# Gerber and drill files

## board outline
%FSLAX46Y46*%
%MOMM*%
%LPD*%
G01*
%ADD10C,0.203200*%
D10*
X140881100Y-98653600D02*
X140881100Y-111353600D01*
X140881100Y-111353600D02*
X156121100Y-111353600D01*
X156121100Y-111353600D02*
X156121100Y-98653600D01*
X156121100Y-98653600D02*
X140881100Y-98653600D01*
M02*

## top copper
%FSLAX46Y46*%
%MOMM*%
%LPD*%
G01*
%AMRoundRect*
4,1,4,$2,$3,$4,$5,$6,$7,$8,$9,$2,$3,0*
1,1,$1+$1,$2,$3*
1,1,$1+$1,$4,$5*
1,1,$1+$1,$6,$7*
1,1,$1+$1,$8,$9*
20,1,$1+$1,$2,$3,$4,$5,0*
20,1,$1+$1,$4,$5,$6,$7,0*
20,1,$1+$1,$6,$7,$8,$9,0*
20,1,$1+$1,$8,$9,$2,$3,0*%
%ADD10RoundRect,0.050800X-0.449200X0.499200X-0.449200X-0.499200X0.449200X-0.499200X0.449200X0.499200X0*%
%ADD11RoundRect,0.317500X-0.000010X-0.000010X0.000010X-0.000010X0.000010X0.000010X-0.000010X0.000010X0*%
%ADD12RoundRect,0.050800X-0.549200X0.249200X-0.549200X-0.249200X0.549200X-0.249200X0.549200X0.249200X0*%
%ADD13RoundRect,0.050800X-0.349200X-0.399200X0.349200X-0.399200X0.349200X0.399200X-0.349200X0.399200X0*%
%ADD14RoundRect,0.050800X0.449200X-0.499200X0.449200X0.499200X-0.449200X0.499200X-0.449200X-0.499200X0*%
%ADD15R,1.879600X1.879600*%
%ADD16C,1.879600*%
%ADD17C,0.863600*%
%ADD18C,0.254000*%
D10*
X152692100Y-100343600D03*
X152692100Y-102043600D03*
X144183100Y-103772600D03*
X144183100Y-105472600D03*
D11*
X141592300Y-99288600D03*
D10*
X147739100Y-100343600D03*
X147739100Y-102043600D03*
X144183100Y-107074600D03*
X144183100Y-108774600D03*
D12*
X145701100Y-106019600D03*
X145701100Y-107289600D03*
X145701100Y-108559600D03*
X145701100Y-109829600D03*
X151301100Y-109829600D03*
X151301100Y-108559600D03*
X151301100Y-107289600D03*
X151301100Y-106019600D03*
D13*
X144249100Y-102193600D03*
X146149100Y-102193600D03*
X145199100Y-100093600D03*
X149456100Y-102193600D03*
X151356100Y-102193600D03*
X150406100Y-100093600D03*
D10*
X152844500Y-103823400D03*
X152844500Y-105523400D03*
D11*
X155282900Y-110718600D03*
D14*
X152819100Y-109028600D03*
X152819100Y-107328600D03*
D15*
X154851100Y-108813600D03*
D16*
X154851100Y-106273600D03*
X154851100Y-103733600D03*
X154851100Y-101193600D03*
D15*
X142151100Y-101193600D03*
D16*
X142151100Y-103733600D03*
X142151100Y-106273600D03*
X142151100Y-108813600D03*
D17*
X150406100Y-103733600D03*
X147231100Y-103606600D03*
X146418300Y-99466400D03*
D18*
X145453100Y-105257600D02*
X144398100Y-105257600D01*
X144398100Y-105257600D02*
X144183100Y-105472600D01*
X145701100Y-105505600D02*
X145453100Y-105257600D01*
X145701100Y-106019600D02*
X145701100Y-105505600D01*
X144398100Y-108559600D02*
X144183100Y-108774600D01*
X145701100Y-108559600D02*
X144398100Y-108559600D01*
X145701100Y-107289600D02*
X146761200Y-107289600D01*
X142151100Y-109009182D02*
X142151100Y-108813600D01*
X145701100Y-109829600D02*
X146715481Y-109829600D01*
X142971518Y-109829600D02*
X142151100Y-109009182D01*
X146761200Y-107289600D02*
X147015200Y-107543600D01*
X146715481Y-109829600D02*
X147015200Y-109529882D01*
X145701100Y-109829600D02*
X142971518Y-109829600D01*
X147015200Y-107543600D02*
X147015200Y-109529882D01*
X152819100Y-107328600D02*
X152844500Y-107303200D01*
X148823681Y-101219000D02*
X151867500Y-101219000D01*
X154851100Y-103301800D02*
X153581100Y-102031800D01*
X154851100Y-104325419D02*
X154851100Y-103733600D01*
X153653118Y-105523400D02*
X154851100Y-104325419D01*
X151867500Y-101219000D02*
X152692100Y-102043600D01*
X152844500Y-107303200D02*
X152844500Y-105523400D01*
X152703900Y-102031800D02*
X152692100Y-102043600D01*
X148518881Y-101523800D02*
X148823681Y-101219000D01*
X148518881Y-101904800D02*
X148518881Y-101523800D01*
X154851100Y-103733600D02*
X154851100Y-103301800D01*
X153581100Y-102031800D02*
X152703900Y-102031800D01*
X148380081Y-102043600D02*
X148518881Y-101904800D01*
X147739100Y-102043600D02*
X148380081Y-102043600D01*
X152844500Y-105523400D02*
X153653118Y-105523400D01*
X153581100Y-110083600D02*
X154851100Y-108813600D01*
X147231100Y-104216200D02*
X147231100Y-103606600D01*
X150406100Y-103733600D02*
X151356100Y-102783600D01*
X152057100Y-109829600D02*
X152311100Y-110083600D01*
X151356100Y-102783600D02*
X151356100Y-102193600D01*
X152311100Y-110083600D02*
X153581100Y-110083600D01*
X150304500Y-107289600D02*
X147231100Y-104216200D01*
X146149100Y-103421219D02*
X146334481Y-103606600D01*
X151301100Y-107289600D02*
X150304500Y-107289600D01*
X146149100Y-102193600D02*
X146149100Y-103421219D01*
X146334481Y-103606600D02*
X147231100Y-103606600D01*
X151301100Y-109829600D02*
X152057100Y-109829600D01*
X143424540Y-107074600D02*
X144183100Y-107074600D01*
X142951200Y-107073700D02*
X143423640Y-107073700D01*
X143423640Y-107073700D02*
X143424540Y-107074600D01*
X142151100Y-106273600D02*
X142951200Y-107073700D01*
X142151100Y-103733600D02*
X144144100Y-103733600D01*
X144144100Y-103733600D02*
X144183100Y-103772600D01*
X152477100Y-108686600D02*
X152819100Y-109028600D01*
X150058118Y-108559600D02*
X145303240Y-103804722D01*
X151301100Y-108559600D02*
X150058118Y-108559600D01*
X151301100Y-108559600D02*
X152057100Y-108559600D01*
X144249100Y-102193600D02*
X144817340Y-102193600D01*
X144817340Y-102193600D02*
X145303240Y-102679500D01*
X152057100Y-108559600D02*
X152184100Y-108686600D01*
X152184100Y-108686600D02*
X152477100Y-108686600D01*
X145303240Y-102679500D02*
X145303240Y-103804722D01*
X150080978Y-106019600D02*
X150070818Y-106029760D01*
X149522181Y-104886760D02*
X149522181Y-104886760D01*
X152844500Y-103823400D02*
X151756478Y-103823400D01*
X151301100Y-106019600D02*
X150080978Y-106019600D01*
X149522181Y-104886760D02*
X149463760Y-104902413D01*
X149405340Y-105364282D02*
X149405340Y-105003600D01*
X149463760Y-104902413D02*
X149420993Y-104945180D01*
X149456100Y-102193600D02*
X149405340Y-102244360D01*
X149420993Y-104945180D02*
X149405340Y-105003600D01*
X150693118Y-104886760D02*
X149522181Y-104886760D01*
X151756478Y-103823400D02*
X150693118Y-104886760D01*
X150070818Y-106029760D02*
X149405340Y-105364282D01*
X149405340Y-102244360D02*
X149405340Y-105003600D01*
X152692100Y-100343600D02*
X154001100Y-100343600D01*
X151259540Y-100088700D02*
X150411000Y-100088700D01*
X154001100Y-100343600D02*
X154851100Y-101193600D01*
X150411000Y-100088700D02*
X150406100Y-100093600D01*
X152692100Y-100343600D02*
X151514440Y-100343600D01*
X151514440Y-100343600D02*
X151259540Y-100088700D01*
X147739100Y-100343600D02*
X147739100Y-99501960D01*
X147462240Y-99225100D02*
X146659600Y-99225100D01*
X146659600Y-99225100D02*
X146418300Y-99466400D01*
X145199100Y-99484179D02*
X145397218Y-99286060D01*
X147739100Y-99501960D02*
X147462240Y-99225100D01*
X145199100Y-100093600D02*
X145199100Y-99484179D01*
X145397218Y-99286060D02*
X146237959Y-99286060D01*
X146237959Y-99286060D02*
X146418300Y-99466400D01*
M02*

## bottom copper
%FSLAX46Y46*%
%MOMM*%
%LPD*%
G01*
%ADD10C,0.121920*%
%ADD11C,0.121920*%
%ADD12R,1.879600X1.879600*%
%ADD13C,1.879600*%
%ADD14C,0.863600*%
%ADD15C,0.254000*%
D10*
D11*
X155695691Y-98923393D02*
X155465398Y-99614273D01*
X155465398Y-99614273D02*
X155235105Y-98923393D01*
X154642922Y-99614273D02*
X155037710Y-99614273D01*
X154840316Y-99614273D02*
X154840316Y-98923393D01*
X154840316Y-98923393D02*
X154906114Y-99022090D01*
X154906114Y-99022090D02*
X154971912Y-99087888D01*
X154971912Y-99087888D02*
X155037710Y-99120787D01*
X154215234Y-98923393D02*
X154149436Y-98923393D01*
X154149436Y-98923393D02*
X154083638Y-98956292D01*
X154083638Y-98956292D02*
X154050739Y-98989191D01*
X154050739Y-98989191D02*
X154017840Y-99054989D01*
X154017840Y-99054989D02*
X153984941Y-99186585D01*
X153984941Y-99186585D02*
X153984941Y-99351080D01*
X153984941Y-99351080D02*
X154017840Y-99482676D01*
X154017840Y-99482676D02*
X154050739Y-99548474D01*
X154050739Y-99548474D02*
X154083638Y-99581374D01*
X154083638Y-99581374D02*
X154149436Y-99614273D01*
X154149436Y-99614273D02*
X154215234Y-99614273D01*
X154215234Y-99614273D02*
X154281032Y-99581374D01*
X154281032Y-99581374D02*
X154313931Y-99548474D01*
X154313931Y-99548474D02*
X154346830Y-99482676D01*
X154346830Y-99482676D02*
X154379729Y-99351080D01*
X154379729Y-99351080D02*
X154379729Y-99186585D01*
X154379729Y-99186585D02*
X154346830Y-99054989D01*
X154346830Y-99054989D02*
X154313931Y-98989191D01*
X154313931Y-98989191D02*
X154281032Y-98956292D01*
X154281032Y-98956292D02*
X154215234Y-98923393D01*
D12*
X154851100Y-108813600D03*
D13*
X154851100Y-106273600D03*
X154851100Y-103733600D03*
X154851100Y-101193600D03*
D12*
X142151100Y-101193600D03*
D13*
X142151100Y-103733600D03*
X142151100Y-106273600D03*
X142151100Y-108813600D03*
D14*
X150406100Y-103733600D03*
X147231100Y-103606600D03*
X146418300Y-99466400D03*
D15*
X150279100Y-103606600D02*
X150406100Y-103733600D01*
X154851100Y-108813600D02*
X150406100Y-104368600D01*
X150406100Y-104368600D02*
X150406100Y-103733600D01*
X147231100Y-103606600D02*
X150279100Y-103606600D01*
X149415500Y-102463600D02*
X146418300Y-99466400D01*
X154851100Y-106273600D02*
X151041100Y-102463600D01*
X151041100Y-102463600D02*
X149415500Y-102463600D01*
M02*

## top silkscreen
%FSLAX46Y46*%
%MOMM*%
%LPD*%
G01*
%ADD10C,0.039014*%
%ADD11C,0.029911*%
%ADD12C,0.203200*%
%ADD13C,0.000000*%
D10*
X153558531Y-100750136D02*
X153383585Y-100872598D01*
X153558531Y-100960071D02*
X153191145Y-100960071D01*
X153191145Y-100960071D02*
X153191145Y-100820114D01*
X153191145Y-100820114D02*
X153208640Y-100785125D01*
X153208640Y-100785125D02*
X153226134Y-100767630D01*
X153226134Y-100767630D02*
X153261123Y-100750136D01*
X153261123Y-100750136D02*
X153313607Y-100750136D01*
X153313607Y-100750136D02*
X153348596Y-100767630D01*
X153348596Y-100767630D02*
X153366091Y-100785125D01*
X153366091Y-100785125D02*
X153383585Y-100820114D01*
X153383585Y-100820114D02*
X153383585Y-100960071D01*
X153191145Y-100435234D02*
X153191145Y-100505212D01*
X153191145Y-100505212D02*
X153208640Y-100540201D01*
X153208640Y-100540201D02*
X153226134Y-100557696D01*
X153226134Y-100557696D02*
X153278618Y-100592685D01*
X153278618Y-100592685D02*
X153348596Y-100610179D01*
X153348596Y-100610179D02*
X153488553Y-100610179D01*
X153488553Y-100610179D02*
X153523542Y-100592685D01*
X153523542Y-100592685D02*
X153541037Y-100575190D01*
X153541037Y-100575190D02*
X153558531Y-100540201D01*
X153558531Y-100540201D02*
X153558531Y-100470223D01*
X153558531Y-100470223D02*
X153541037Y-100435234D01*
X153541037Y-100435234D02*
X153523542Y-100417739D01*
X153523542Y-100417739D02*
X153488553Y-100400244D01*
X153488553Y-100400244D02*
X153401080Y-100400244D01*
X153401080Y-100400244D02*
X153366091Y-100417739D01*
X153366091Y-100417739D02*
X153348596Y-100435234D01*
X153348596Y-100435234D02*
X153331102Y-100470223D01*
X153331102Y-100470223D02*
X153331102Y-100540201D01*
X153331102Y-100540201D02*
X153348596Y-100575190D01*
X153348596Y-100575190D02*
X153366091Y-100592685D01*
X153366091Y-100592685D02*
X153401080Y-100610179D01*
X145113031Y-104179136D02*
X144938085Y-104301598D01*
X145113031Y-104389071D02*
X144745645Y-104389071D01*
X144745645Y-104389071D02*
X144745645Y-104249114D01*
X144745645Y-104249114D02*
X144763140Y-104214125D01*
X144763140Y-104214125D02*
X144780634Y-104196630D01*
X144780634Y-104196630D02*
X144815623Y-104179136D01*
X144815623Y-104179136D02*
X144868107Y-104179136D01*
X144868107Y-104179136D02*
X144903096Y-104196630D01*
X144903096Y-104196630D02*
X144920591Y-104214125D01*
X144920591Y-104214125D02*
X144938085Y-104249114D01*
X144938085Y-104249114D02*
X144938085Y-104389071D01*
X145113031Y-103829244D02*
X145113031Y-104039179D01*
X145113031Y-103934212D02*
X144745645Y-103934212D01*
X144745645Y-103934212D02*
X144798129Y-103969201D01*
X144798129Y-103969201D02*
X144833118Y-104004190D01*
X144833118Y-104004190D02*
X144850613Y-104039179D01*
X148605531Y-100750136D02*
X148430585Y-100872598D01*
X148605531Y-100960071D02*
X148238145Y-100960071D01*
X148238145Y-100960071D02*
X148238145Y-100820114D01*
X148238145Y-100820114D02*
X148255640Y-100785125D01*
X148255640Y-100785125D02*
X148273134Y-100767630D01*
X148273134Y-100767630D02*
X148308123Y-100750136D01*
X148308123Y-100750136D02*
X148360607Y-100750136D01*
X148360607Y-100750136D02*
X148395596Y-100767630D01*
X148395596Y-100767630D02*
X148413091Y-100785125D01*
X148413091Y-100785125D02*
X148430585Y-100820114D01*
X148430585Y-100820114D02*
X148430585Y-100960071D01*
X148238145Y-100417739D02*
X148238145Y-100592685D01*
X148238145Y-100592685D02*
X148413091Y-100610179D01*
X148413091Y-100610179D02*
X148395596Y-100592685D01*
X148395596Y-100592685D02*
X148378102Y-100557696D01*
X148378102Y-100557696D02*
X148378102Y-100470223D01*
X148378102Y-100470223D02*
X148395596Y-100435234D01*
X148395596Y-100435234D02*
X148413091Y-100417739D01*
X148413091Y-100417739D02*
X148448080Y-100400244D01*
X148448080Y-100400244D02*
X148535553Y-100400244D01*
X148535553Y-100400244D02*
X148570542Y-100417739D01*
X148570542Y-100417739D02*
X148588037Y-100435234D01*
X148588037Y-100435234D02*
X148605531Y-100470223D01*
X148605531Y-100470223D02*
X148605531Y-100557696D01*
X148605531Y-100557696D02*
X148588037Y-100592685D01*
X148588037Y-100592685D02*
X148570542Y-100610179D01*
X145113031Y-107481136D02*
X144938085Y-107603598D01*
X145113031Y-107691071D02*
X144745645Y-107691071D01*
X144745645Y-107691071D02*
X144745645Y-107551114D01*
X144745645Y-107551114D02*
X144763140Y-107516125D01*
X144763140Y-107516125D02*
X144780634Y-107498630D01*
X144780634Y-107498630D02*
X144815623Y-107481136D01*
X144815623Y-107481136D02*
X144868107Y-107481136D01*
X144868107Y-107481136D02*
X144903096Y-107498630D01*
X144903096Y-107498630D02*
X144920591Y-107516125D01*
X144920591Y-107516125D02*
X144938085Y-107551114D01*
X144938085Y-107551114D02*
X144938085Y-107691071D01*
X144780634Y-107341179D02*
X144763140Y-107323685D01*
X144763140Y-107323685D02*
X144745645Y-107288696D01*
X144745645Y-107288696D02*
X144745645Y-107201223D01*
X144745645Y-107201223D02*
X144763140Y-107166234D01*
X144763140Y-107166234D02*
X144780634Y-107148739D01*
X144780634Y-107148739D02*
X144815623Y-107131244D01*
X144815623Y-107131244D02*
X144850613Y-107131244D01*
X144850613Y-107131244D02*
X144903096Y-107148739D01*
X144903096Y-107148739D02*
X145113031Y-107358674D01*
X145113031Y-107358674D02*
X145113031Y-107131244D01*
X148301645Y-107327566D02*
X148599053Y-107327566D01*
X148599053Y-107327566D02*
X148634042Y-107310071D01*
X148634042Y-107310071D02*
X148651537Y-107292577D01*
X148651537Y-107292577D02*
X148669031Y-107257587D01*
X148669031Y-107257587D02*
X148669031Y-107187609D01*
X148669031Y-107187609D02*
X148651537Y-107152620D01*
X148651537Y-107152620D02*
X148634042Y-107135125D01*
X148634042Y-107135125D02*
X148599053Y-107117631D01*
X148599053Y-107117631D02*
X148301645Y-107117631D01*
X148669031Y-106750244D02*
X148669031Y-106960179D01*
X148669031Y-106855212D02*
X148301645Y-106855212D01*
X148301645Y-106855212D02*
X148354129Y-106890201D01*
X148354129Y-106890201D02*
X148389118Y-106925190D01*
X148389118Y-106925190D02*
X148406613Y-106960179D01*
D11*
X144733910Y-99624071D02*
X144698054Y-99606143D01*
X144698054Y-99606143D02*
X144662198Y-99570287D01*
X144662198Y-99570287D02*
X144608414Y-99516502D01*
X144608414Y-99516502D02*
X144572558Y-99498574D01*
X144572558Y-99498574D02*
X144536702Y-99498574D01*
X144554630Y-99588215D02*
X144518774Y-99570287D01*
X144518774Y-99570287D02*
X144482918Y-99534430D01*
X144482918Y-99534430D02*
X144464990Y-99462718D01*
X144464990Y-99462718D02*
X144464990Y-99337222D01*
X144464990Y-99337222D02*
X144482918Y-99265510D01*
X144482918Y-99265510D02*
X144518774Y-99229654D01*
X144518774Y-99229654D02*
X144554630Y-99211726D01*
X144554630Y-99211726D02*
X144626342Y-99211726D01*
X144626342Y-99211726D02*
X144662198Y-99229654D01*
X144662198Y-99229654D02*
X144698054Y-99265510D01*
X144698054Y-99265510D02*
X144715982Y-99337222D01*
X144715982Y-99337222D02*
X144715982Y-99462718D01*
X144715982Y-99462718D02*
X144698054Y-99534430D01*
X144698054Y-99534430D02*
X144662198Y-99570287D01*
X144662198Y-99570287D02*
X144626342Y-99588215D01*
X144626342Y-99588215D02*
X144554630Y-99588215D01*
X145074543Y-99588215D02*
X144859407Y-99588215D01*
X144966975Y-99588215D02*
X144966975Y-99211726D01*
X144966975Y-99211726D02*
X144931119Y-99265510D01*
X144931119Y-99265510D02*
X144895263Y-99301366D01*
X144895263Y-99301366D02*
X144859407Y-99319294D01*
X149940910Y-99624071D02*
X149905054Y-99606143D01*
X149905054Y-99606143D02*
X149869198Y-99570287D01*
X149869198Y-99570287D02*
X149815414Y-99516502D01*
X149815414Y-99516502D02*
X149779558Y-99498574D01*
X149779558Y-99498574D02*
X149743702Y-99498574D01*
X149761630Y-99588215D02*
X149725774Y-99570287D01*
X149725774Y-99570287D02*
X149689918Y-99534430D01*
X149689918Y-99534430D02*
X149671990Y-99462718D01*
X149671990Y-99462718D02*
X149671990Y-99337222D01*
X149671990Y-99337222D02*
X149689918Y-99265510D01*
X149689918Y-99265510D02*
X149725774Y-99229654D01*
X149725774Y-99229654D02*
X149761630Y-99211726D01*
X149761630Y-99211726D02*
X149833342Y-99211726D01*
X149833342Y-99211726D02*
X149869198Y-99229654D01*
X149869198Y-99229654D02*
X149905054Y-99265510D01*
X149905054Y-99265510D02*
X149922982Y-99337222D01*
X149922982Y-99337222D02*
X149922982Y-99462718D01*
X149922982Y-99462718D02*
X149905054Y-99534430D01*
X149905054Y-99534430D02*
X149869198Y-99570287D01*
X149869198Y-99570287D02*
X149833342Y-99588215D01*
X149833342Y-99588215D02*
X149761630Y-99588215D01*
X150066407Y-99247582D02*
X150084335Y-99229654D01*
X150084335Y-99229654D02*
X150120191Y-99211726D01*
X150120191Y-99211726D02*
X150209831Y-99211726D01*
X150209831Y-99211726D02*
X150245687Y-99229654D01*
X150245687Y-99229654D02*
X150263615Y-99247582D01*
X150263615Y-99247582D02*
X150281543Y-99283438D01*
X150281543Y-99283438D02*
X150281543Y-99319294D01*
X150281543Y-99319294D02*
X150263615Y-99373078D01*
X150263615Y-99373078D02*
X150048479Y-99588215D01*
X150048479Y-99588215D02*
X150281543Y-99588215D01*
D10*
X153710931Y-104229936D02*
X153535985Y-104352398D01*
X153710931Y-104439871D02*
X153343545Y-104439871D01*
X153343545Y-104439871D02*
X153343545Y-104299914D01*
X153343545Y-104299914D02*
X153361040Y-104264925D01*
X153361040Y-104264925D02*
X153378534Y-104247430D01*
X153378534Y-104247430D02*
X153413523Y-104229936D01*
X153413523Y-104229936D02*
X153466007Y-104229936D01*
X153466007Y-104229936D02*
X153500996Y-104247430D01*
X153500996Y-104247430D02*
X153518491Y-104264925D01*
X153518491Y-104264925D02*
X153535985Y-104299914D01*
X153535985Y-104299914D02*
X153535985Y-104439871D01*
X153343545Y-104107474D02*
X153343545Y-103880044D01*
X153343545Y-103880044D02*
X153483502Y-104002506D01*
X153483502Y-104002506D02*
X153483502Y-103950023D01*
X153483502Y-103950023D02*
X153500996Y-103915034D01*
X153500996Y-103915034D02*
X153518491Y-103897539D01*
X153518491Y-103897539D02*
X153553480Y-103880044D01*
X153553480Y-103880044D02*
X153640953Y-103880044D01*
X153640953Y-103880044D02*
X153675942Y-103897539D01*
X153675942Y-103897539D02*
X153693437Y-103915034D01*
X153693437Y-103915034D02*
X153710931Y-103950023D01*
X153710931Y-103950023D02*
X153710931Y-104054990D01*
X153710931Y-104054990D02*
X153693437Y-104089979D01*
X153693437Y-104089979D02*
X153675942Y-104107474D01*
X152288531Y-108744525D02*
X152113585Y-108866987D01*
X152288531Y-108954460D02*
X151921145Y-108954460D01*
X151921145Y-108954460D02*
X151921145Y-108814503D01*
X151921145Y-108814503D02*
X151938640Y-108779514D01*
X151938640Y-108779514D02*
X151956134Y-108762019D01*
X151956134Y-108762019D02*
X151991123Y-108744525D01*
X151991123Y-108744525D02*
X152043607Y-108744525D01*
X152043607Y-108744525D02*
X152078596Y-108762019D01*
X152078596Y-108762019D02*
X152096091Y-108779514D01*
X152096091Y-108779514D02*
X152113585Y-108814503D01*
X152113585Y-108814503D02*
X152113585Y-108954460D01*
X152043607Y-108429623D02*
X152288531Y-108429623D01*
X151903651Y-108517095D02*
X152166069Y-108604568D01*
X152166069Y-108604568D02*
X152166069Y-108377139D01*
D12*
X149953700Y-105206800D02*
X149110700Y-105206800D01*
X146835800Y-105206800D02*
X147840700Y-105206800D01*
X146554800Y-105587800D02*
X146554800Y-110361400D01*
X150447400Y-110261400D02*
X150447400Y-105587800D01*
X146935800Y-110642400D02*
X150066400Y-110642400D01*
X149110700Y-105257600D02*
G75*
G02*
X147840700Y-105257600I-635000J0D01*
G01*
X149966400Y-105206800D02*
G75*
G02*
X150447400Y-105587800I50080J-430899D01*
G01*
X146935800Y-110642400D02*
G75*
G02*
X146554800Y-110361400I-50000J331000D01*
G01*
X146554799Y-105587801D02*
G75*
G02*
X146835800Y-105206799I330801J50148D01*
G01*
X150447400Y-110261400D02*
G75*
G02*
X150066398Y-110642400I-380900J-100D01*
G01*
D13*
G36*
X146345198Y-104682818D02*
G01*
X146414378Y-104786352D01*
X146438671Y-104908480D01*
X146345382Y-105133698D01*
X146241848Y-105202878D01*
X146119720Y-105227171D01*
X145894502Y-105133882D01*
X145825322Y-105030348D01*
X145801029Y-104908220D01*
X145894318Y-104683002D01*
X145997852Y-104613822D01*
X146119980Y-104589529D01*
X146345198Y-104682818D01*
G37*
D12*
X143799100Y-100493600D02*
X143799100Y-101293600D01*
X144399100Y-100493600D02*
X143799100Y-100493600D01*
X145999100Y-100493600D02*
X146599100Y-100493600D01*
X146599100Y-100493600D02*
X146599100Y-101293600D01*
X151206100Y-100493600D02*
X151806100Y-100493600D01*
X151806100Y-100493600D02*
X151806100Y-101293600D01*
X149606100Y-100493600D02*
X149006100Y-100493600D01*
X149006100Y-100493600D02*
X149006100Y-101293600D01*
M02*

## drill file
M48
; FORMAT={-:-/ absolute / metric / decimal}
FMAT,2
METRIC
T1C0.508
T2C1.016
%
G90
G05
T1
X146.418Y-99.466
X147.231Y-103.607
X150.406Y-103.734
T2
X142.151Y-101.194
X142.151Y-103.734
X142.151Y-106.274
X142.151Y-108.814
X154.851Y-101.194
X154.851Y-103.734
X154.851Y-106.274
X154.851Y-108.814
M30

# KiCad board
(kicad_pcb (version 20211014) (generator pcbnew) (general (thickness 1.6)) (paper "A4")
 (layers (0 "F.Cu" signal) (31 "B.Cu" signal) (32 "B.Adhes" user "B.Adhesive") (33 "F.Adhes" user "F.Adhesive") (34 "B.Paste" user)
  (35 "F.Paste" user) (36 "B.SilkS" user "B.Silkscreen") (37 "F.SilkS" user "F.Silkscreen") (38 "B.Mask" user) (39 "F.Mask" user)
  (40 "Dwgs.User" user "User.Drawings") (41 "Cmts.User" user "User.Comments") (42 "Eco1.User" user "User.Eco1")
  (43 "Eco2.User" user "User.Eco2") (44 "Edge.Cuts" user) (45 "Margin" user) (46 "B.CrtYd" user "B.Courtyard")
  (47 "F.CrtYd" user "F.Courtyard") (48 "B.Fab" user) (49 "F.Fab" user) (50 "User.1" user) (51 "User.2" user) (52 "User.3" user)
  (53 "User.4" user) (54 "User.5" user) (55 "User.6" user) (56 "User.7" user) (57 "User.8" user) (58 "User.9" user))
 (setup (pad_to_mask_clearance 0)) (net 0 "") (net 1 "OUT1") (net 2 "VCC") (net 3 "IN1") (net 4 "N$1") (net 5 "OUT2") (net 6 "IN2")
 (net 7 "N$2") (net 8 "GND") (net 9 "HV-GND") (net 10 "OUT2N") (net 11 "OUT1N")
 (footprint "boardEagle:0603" (layer "F.Cu") (at 152.6921 101.1936 -90)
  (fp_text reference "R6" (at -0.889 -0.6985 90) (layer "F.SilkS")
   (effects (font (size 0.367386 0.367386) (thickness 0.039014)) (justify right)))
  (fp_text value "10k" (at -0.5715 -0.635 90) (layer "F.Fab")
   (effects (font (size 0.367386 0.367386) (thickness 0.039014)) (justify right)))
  (pad "1" smd roundrect (at -0.85 0 270) (size 1.1 1) (layers "F.Cu" "F.Paste" "F.Mask") (roundrect_rratio 0.0508) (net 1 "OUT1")
   (solder_mask_margin 0.0762))
  (pad "2" smd roundrect (at 0.85 0 270) (size 1.1 1) (layers "F.Cu" "F.Paste" "F.Mask") (roundrect_rratio 0.0508) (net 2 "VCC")
   (solder_mask_margin 0.0762)))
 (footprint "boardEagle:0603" (layer "F.Cu") (at 144.1831 104.6226 -90)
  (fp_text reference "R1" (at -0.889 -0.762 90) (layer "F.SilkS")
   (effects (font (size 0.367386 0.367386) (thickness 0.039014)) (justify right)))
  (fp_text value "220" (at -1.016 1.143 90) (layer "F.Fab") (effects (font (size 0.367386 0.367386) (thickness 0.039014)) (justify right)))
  (pad "1" smd roundrect (at -0.85 0 270) (size 1.1 1) (layers "F.Cu" "F.Paste" "F.Mask") (roundrect_rratio 0.0508) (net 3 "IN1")
   (solder_mask_margin 0.0762))
  (pad "2" smd roundrect (at 0.85 0 270) (size 1.1 1) (layers "F.Cu" "F.Paste" "F.Mask") (roundrect_rratio 0.0508) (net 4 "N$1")
   (solder_mask_margin 0.0762)))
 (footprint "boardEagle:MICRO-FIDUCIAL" (layer "F.Cu") (at 141.5923 99.2886)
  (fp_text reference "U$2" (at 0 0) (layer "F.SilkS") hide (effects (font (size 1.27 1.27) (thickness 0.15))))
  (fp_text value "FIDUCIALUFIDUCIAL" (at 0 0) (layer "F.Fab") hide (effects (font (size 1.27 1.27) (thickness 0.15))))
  (pad "1" smd roundrect (at 0 0) (size 0.635 0.635) (layers "F.Cu" "F.Mask") (roundrect_rratio 0.5) (solder_mask_margin 0.0762)))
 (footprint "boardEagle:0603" (layer "F.Cu") (at 147.7391 101.1936 -90)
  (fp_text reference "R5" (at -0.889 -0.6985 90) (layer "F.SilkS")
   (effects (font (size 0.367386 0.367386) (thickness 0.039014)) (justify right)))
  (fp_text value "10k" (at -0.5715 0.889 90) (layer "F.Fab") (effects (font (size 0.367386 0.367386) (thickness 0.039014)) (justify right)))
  (pad "1" smd roundrect (at -0.85 0 270) (size 1.1 1) (layers "F.Cu" "F.Paste" "F.Mask") (roundrect_rratio 0.0508) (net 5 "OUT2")
   (solder_mask_margin 0.0762))
  (pad "2" smd roundrect (at 0.85 0 270) (size 1.1 1) (layers "F.Cu" "F.Paste" "F.Mask") (roundrect_rratio 0.0508) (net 2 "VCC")
   (solder_mask_margin 0.0762)))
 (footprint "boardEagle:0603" (layer "F.Cu") (at 144.1831 107.9246 -90)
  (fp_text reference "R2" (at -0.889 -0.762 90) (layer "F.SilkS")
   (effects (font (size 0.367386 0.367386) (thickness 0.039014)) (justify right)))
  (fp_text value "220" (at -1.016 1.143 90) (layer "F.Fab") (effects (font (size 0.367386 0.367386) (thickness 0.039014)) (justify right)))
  (pad "1" smd roundrect (at -0.85 0 270) (size 1.1 1) (layers "F.Cu" "F.Paste" "F.Mask") (roundrect_rratio 0.0508) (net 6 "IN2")
   (solder_mask_margin 0.0762))
  (pad "2" smd roundrect (at 0.85 0 270) (size 1.1 1) (layers "F.Cu" "F.Paste" "F.Mask") (roundrect_rratio 0.0508) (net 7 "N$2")
   (solder_mask_margin 0.0762)))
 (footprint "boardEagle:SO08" (layer "F.Cu") (at 148.5011 107.9246 -90)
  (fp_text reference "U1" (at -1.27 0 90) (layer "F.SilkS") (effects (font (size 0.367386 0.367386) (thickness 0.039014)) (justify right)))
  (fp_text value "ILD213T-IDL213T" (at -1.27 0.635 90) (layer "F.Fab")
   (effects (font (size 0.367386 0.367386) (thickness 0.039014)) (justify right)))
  (fp_line (start -2.7178 -1.4526) (end -2.7178 -0.6096) (layer "F.SilkS") (width 0.2032))
  (fp_line (start -2.7178 1.6653) (end -2.7178 0.6604) (layer "F.SilkS") (width 0.2032))
  (fp_line (start -2.3368 1.9463) (end 2.4368 1.9463) (layer "F.SilkS") (width 0.2032))
  (fp_line (start 2.3368 -1.9463) (end -2.3368 -1.9463) (layer "F.SilkS") (width 0.2032))
  (fp_line (start 2.7178 1.5653) (end 2.7178 -1.5653) (layer "F.SilkS") (width 0.2032))
  (fp_arc (start -2.667 -0.6096) (mid -2.032 0.0254) (end -2.667 0.6604) (layer "F.SilkS") (width 0.2032))
  (fp_arc (start -2.7178 -1.4653) (mid -2.626948 -1.784731) (end -2.3368 -1.9463) (layer "F.SilkS") (width 0.2032))
  (fp_arc (start 2.7178 1.5653) (mid 2.656208 1.813997) (end 2.4368 1.9463) (layer "F.SilkS") (width 0.2032))
  (fp_arc (start -2.336799 1.946301) (mid -2.58554 1.884767) (end -2.7178 1.6653) (layer "F.SilkS") (width 0.2032))
  (fp_arc (start 2.3368 -1.9463) (mid 2.606237 -1.834736) (end 2.7178 -1.565298) (layer "F.SilkS") (width 0.2032))
  (fp_poly
   (pts (xy -2.790902 2.155718) (xy -2.721722 2.259252) (xy -2.697429 2.38138) (xy -2.790718 2.606598) (xy -2.894252 2.675778)
    (xy -3.01638 2.700071) (xy -3.241598 2.606782) (xy -3.310778 2.503248) (xy -3.335071 2.38112) (xy -3.241782 2.155902)
    (xy -3.138248 2.086722) (xy -3.01612 2.062429))
   (layer "F.SilkS") (width 0) (fill solid))
  (pad "1" smd roundrect (at -1.905 2.8 270) (size 0.6 1.2) (layers "F.Cu" "F.Paste" "F.Mask") (roundrect_rratio 0.08466666667)
   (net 4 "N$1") (solder_mask_margin 0.0762))
  (pad "2" smd roundrect (at -0.635 2.8 270) (size 0.6 1.2) (layers "F.Cu" "F.Paste" "F.Mask") (roundrect_rratio 0.08466666667)
   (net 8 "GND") (solder_mask_margin 0.0762))
  (pad "3" smd roundrect (at 0.635 2.8 270) (size 0.6 1.2) (layers "F.Cu" "F.Paste" "F.Mask") (roundrect_rratio 0.08466666667) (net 7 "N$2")
   (solder_mask_margin 0.0762))
  (pad "4" smd roundrect (at 1.905 2.8 270) (size 0.6 1.2) (layers "F.Cu" "F.Paste" "F.Mask") (roundrect_rratio 0.08466666667) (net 8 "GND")
   (solder_mask_margin 0.0762))
  (pad "5" smd roundrect (at 1.905 -2.8 270) (size 0.6 1.2) (layers "F.Cu" "F.Paste" "F.Mask") (roundrect_rratio 0.08466666667)
   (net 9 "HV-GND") (solder_mask_margin 0.0762))
  (pad "6" smd roundrect (at 0.635 -2.8 270) (size 0.6 1.2) (layers "F.Cu" "F.Paste" "F.Mask") (roundrect_rratio 0.08466666667)
   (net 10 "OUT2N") (solder_mask_margin 0.0762))
  (pad "7" smd roundrect (at -0.635 -2.8 270) (size 0.6 1.2) (layers "F.Cu" "F.Paste" "F.Mask") (roundrect_rratio 0.08466666667)
   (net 9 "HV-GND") (solder_mask_margin 0.0762))
  (pad "8" smd roundrect (at -1.905 -2.8 270) (size 0.6 1.2) (layers "F.Cu" "F.Paste" "F.Mask") (roundrect_rratio 0.08466666667)
   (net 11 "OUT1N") (solder_mask_margin 0.0762)))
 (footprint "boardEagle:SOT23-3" (layer "F.Cu") (at 145.1991 101.1936)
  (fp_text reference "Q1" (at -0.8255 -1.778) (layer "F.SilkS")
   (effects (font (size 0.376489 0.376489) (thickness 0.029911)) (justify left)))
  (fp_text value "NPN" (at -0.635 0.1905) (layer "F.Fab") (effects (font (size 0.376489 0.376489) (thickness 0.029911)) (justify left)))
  (fp_line (start -1.4 -0.7) (end -1.4 0.1) (layer "F.SilkS") (width 0.2032))
  (fp_line (start -0.8 -0.7) (end -1.4 -0.7) (layer "F.SilkS") (width 0.2032))
  (fp_line (start 0.8 -0.7) (end 1.4 -0.7) (layer "F.SilkS") (width 0.2032))
  (fp_line (start 1.4 -0.7) (end 1.4 0.1) (layer "F.SilkS") (width 0.2032))
  (pad "1" smd roundrect (at -0.95 1) (size 0.8 0.9) (layers "F.Cu" "F.Paste" "F.Mask") (roundrect_rratio 0.0635) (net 10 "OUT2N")
   (solder_mask_margin 0.0762))
  (pad "2" smd roundrect (at 0.95 1) (size 0.8 0.9) (layers "F.Cu" "F.Paste" "F.Mask") (roundrect_rratio 0.0635) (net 9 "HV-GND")
   (solder_mask_margin 0.0762))
  (pad "3" smd roundrect (at 0 -1.1) (size 0.8 0.9) (layers "F.Cu" "F.Paste" "F.Mask") (roundrect_rratio 0.0635) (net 5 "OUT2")
   (solder_mask_margin 0.0762)))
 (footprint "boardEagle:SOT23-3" (layer "F.Cu") (at 150.4061 101.1936)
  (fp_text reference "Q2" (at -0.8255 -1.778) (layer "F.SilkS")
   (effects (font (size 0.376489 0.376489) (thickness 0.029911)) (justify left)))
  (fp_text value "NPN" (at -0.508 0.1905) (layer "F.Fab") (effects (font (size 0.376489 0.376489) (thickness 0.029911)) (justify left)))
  (fp_line (start 0.8 -0.7) (end 1.4 -0.7) (layer "F.SilkS") (width 0.2032))
  (fp_line (start 1.4 -0.7) (end 1.4 0.1) (layer "F.SilkS") (width 0.2032))
  (fp_line (start -0.8 -0.7) (end -1.4 -0.7) (layer "F.SilkS") (width 0.2032))
  (fp_line (start -1.4 -0.7) (end -1.4 0.1) (layer "F.SilkS") (width 0.2032))
  (pad "1" smd roundrect (at -0.95 1) (size 0.8 0.9) (layers "F.Cu" "F.Paste" "F.Mask") (roundrect_rratio 0.0635) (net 11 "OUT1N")
   (solder_mask_margin 0.0762))
  (pad "2" smd roundrect (at 0.95 1) (size 0.8 0.9) (layers "F.Cu" "F.Paste" "F.Mask") (roundrect_rratio 0.0635) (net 9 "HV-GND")
   (solder_mask_margin 0.0762))
  (pad "3" smd roundrect (at 0 -1.1) (size 0.8 0.9) (layers "F.Cu" "F.Paste" "F.Mask") (roundrect_rratio 0.0635) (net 1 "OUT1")
   (solder_mask_margin 0.0762)))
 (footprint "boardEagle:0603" (layer "F.Cu") (at 152.8445 104.6734 -90)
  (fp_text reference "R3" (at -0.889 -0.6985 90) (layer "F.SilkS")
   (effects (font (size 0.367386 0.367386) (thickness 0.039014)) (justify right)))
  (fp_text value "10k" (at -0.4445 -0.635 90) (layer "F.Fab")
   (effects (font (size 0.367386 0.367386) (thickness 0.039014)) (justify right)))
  (pad "1" smd roundrect (at -0.85 0 270) (size 1.1 1) (layers "F.Cu" "F.Paste" "F.Mask") (roundrect_rratio 0.0508) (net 11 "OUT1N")
   (solder_mask_margin 0.0762))
  (pad "2" smd roundrect (at 0.85 0 270) (size 1.1 1) (layers "F.Cu" "F.Paste" "F.Mask") (roundrect_rratio 0.0508) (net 2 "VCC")
   (solder_mask_margin 0.0762)))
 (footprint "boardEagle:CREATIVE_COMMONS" (layer "F.Cu") (at 118.159513 124.0536)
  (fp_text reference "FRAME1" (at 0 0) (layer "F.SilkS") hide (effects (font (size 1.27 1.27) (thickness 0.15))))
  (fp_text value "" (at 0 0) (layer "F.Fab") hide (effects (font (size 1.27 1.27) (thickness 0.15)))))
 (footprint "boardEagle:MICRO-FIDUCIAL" (layer "F.Cu") (at 155.2829 110.7186)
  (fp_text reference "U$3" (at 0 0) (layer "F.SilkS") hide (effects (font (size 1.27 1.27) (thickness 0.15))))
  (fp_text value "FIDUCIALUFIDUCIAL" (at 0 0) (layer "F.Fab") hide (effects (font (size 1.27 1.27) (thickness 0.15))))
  (pad "1" smd roundrect (at 0 0) (size 0.635 0.635) (layers "F.Cu" "F.Mask") (roundrect_rratio 0.5) (solder_mask_margin 0.0762)))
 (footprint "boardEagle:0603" (layer "F.Cu") (at 152.8191 108.1786 90)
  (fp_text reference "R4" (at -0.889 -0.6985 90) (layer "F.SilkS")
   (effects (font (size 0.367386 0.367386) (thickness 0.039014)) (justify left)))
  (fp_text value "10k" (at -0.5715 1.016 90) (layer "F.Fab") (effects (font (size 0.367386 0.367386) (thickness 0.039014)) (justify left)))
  (pad "1" smd roundrect (at -0.85 0 90) (size 1.1 1) (layers "F.Cu" "F.Paste" "F.Mask") (roundrect_rratio 0.0508) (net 10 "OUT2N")
   (solder_mask_margin 0.0762))
  (pad "2" smd roundrect (at 0.85 0 90) (size 1.1 1) (layers "F.Cu" "F.Paste" "F.Mask") (roundrect_rratio 0.0508) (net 2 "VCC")
   (solder_mask_margin 0.0762)))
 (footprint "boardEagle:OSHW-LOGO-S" (layer "B.Cu") (at 148.5044 102.902257 180)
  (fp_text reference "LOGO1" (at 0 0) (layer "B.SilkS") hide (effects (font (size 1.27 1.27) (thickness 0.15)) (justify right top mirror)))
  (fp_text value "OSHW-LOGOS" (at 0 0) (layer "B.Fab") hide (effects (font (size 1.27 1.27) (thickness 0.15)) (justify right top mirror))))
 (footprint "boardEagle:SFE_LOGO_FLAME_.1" (layer "B.Cu") (at 149.591521 107.603291 180)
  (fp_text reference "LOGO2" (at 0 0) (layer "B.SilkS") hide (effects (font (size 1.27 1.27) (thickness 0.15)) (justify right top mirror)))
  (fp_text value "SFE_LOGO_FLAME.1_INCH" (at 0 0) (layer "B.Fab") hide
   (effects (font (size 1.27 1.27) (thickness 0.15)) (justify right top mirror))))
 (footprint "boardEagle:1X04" (layer "B.Cu") (at 154.8511 108.8136 90)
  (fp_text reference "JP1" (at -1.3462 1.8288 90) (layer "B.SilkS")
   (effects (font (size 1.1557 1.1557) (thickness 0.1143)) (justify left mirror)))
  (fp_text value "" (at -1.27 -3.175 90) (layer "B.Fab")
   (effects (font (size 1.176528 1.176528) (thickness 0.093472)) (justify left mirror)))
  (pad "1" thru_hole rect (at 0 0) (size 1.8796 1.8796) (drill 1.016) (layers *.Cu *.Mask) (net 9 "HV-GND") (solder_mask_margin 0.0762))
  (pad "2" thru_hole circle (at 2.54 0) (size 1.8796 1.8796) (drill 1.016) (layers *.Cu *.Mask) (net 5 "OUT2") (solder_mask_margin 0.0762))
  (pad "3" thru_hole circle (at 5.08 0) (size 1.8796 1.8796) (drill 1.016) (layers *.Cu *.Mask) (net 2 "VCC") (solder_mask_margin 0.0762))
  (pad "4" thru_hole circle (at 7.62 0) (size 1.8796 1.8796) (drill 1.016) (layers *.Cu *.Mask) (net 1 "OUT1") (solder_mask_margin 0.0762)))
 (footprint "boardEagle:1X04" (layer "B.Cu") (at 142.1511 101.1936 -90)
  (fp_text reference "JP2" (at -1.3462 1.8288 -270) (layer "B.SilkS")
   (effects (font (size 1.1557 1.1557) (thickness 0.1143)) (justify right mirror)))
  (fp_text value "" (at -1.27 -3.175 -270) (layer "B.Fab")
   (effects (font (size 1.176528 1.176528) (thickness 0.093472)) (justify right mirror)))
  (pad "1" thru_hole rect (at 0 0 180) (size 1.8796 1.8796) (drill 1.016) (layers *.Cu *.Mask) (solder_mask_margin 0.0762))
  (pad "2" thru_hole circle (at 2.54 0 180) (size 1.8796 1.8796) (drill 1.016) (layers *.Cu *.Mask) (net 3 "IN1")
   (solder_mask_margin 0.0762))
  (pad "3" thru_hole circle (at 5.08 0 180) (size 1.8796 1.8796) (drill 1.016) (layers *.Cu *.Mask) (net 6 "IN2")
   (solder_mask_margin 0.0762))
  (pad "4" thru_hole circle (at 7.62 0 180) (size 1.8796 1.8796) (drill 1.016) (layers *.Cu *.Mask) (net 8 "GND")
   (solder_mask_margin 0.0762)))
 (gr_line (start 140.8811 98.6536) (end 140.8811 111.3536) (layer "Edge.Cuts") (width 0.2032))
 (gr_line (start 140.8811 111.3536) (end 156.1211 111.3536) (layer "Edge.Cuts") (width 0.2032))
 (gr_line (start 156.1211 111.3536) (end 156.1211 98.6536) (layer "Edge.Cuts") (width 0.2032))
 (gr_line (start 156.1211 98.6536) (end 140.8811 98.6536) (layer "Edge.Cuts") (width 0.2032))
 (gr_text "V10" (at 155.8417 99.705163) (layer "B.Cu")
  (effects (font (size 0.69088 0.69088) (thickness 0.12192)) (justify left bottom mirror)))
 (segment (start 145.4531 105.2576) (end 144.3981 105.2576) (width 0.254) (layer "F.Cu") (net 4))
 (segment (start 144.3981 105.2576) (end 144.1831 105.4726) (width 0.254) (layer "F.Cu") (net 4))
 (segment (start 145.7011 105.5056) (end 145.4531 105.2576) (width 0.254) (layer "F.Cu") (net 4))
 (segment (start 145.7011 106.0196) (end 145.7011 105.5056) (width 0.254) (layer "F.Cu") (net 4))
 (segment (start 144.3981 108.5596) (end 144.1831 108.7746) (width 0.254) (layer "F.Cu") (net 7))
 (segment (start 145.7011 108.5596) (end 144.3981 108.5596) (width 0.254) (layer "F.Cu") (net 7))
 (segment (start 145.7011 107.2896) (end 146.7612 107.2896) (width 0.254) (layer "F.Cu") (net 8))
 (segment (start 142.1511 109.009182) (end 142.1511 108.8136) (width 0.254) (layer "F.Cu") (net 8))
 (segment (start 145.7011 109.8296) (end 146.715481 109.8296) (width 0.254) (layer "F.Cu") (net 8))
 (segment (start 142.971518 109.8296) (end 142.1511 109.009182) (width 0.254) (layer "F.Cu") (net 8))
 (segment (start 146.7612 107.2896) (end 147.0152 107.5436) (width 0.254) (layer "F.Cu") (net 8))
 (segment (start 146.715481 109.8296) (end 147.0152 109.529882) (width 0.254) (layer "F.Cu") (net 8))
 (segment (start 145.7011 109.8296) (end 142.971518 109.8296) (width 0.254) (layer "F.Cu") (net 8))
 (segment (start 147.0152 107.5436) (end 147.0152 109.529882) (width 0.254) (layer "F.Cu") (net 8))
 (segment (start 152.8191 107.3286) (end 152.8445 107.3032) (width 0.254) (layer "F.Cu") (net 2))
 (segment (start 148.823681 101.219) (end 151.8675 101.219) (width 0.254) (layer "F.Cu") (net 2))
 (segment (start 154.8511 103.3018) (end 153.5811 102.0318) (width 0.254) (layer "F.Cu") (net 2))
 (segment (start 154.8511 104.325419) (end 154.8511 103.7336) (width 0.254) (layer "F.Cu") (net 2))
 (segment (start 153.653118 105.5234) (end 154.8511 104.325419) (width 0.254) (layer "F.Cu") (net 2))
 (segment (start 151.8675 101.219) (end 152.6921 102.0436) (width 0.254) (layer "F.Cu") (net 2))
 (segment (start 152.8445 107.3032) (end 152.8445 105.5234) (width 0.254) (layer "F.Cu") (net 2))
 (segment (start 152.7039 102.0318) (end 152.6921 102.0436) (width 0.254) (layer "F.Cu") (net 2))
 (segment (start 148.518881 101.5238) (end 148.823681 101.219) (width 0.254) (layer "F.Cu") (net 2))
 (segment (start 148.518881 101.9048) (end 148.518881 101.5238) (width 0.254) (layer "F.Cu") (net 2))
 (segment (start 154.8511 103.7336) (end 154.8511 103.3018) (width 0.254) (layer "F.Cu") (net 2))
 (segment (start 153.5811 102.0318) (end 152.7039 102.0318) (width 0.254) (layer "F.Cu") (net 2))
 (segment (start 148.380081 102.0436) (end 148.518881 101.9048) (width 0.254) (layer "F.Cu") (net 2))
 (segment (start 147.7391 102.0436) (end 148.380081 102.0436) (width 0.254) (layer "F.Cu") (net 2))
 (segment (start 152.8445 105.5234) (end 153.653118 105.5234) (width 0.254) (layer "F.Cu") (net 2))
 (segment (start 153.5811 110.0836) (end 154.8511 108.8136) (width 0.254) (layer "F.Cu") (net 9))
 (segment (start 147.2311 104.2162) (end 147.2311 103.6066) (width 0.254) (layer "F.Cu") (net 9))
 (segment (start 150.4061 103.7336) (end 151.3561 102.7836) (width 0.254) (layer "F.Cu") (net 9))
 (segment (start 152.0571 109.8296) (end 152.3111 110.0836) (width 0.254) (layer "F.Cu") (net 9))
 (segment (start 151.3561 102.7836) (end 151.3561 102.1936) (width 0.254) (layer "F.Cu") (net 9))
 (segment (start 152.3111 110.0836) (end 153.5811 110.0836) (width 0.254) (layer "F.Cu") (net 9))
 (segment (start 150.3045 107.2896) (end 147.2311 104.2162) (width 0.254) (layer "F.Cu") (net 9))
 (segment (start 146.1491 103.421219) (end 146.334481 103.6066) (width 0.254) (layer "F.Cu") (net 9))
 (segment (start 151.3011 107.2896) (end 150.3045 107.2896) (width 0.254) (layer "F.Cu") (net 9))
 (segment (start 146.1491 102.1936) (end 146.1491 103.421219) (width 0.254) (layer "F.Cu") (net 9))
 (segment (start 146.334481 103.6066) (end 147.2311 103.6066) (width 0.254) (layer "F.Cu") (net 9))
 (segment (start 151.3011 109.8296) (end 152.0571 109.8296) (width 0.254) (layer "F.Cu") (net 9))
 (via (at 150.4061 103.7336) (size 0.8636) (drill 0.508) (layers "F.Cu" "B.Cu") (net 9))
 (via (at 147.2311 103.6066) (size 0.8636) (drill 0.508) (layers "F.Cu" "B.Cu") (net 9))
 (segment (start 150.2791 103.6066) (end 150.4061 103.7336) (width 0.254) (layer "B.Cu") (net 9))
 (segment (start 154.8511 108.8136) (end 150.4061 104.3686) (width 0.254) (layer "B.Cu") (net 9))
 (segment (start 150.4061 104.3686) (end 150.4061 103.7336) (width 0.254) (layer "B.Cu") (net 9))
 (segment (start 147.2311 103.6066) (end 150.2791 103.6066) (width 0.254) (layer "B.Cu") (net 9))
 (segment (start 143.42454 107.0746) (end 144.1831 107.0746) (width 0.254) (layer "F.Cu") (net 6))
 (segment (start 142.9512 107.0737) (end 143.42364 107.0737) (width 0.254) (layer "F.Cu") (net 6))
 (segment (start 143.42364 107.0737) (end 143.42454 107.0746) (width 0.254) (layer "F.Cu") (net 6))
 (segment (start 142.1511 106.2736) (end 142.9512 107.0737) (width 0.254) (layer "F.Cu") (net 6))
 (segment (start 142.1511 103.7336) (end 144.1441 103.7336) (width 0.254) (layer "F.Cu") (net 3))
 (segment (start 144.1441 103.7336) (end 144.1831 103.7726) (width 0.254) (layer "F.Cu") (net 3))
 (segment (start 152.4771 108.6866) (end 152.8191 109.0286) (width 0.254) (layer "F.Cu") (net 10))
 (segment (start 150.058118 108.5596) (end 145.30324 103.804722) (width 0.254) (layer "F.Cu") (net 10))
 (segment (start 151.3011 108.5596) (end 150.058118 108.5596) (width 0.254) (layer "F.Cu") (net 10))
 (segment (start 151.3011 108.5596) (end 152.0571 108.5596) (width 0.254) (layer "F.Cu") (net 10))
 (segment (start 144.2491 102.1936) (end 144.81734 102.1936) (width 0.254) (layer "F.Cu") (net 10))
 (segment (start 144.81734 102.1936) (end 145.30324 102.6795) (width 0.254) (layer "F.Cu") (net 10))
 (segment (start 152.0571 108.5596) (end 152.1841 108.6866) (width 0.254) (layer "F.Cu") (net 10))
 (segment (start 152.1841 108.6866) (end 152.4771 108.6866) (width 0.254) (layer "F.Cu") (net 10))
 (segment (start 145.30324 102.6795) (end 145.30324 103.804722) (width 0.254) (layer "F.Cu") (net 10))
 (segment (start 150.080978 106.0196) (end 150.070818 106.02976) (width 0.254) (layer "F.Cu") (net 11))
 (segment (start 149.522181 104.88676) (end 149.522181 104.88676) (width 0.254) (layer "F.Cu") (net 11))
 (segment (start 152.8445 103.8234) (end 151.756478 103.8234) (width 0.254) (layer "F.Cu") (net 11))
 (segment (start 151.3011 106.0196) (end 150.080978 106.0196) (width 0.254) (layer "F.Cu") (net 11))
 (segment (start 149.522181 104.88676) (end 149.46376 104.902413) (width 0.254) (layer "F.Cu") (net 11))
 (segment (start 149.40534 105.364282) (end 149.40534 105.0036) (width 0.254) (layer "F.Cu") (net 11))
 (segment (start 149.46376 104.902413) (end 149.420993 104.94518) (width 0.254) (layer "F.Cu") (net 11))
 (segment (start 149.4561 102.1936) (end 149.40534 102.24436) (width 0.254) (layer "F.Cu") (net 11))
 (segment (start 149.420993 104.94518) (end 149.40534 105.0036) (width 0.254) (layer "F.Cu") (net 11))
 (segment (start 150.693118 104.88676) (end 149.522181 104.88676) (width 0.254) (layer "F.Cu") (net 11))
 (segment (start 151.756478 103.8234) (end 150.693118 104.88676) (width 0.254) (layer "F.Cu") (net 11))
 (segment (start 150.070818 106.02976) (end 149.40534 105.364282) (width 0.254) (layer "F.Cu") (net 11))
 (segment (start 149.40534 102.24436) (end 149.40534 105.0036) (width 0.254) (layer "F.Cu") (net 11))
 (segment (start 152.6921 100.3436) (end 154.0011 100.3436) (width 0.254) (layer "F.Cu") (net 1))
 (segment (start 151.25954 100.0887) (end 150.411 100.0887) (width 0.254) (layer "F.Cu") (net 1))
 (segment (start 154.0011 100.3436) (end 154.8511 101.1936) (width 0.254) (layer "F.Cu") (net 1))
 (segment (start 150.411 100.0887) (end 150.4061 100.0936) (width 0.254) (layer "F.Cu") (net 1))
 (segment (start 152.6921 100.3436) (end 151.51444 100.3436) (width 0.254) (layer "F.Cu") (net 1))
 (segment (start 151.51444 100.3436) (end 151.25954 100.0887) (width 0.254) (layer "F.Cu") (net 1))
 (segment (start 147.7391 100.3436) (end 147.7391 99.50196) (width 0.254) (layer "F.Cu") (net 5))
 (segment (start 147.46224 99.2251) (end 146.6596 99.2251) (width 0.254) (layer "F.Cu") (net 5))
 (segment (start 146.6596 99.2251) (end 146.4183 99.4664) (width 0.254) (layer "F.Cu") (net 5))
 (segment (start 145.1991 99.484179) (end 145.397218 99.28606) (width 0.254) (layer "F.Cu") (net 5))
 (segment (start 147.7391 99.50196) (end 147.46224 99.2251) (width 0.254) (layer "F.Cu") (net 5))
 (segment (start 145.1991 100.0936) (end 145.1991 99.484179) (width 0.254) (layer "F.Cu") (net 5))
 (segment (start 145.397218 99.28606) (end 146.237959 99.28606) (width 0.254) (layer "F.Cu") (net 5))
 (segment (start 146.237959 99.28606) (end 146.4183 99.4664) (width 0.254) (layer "F.Cu") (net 5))
 (via (at 146.4183 99.4664) (size 0.8636) (drill 0.508) (layers "F.Cu" "B.Cu") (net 5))
 (segment (start 149.4155 102.4636) (end 146.4183 99.4664) (width 0.254) (layer "B.Cu") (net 5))
 (segment (start 154.8511 106.2736) (end 151.0411 102.4636) (width 0.254) (layer "B.Cu") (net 5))
 (segment (start 151.0411 102.4636) (end 149.4155 102.4636) (width 0.254) (layer "B.Cu") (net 5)))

